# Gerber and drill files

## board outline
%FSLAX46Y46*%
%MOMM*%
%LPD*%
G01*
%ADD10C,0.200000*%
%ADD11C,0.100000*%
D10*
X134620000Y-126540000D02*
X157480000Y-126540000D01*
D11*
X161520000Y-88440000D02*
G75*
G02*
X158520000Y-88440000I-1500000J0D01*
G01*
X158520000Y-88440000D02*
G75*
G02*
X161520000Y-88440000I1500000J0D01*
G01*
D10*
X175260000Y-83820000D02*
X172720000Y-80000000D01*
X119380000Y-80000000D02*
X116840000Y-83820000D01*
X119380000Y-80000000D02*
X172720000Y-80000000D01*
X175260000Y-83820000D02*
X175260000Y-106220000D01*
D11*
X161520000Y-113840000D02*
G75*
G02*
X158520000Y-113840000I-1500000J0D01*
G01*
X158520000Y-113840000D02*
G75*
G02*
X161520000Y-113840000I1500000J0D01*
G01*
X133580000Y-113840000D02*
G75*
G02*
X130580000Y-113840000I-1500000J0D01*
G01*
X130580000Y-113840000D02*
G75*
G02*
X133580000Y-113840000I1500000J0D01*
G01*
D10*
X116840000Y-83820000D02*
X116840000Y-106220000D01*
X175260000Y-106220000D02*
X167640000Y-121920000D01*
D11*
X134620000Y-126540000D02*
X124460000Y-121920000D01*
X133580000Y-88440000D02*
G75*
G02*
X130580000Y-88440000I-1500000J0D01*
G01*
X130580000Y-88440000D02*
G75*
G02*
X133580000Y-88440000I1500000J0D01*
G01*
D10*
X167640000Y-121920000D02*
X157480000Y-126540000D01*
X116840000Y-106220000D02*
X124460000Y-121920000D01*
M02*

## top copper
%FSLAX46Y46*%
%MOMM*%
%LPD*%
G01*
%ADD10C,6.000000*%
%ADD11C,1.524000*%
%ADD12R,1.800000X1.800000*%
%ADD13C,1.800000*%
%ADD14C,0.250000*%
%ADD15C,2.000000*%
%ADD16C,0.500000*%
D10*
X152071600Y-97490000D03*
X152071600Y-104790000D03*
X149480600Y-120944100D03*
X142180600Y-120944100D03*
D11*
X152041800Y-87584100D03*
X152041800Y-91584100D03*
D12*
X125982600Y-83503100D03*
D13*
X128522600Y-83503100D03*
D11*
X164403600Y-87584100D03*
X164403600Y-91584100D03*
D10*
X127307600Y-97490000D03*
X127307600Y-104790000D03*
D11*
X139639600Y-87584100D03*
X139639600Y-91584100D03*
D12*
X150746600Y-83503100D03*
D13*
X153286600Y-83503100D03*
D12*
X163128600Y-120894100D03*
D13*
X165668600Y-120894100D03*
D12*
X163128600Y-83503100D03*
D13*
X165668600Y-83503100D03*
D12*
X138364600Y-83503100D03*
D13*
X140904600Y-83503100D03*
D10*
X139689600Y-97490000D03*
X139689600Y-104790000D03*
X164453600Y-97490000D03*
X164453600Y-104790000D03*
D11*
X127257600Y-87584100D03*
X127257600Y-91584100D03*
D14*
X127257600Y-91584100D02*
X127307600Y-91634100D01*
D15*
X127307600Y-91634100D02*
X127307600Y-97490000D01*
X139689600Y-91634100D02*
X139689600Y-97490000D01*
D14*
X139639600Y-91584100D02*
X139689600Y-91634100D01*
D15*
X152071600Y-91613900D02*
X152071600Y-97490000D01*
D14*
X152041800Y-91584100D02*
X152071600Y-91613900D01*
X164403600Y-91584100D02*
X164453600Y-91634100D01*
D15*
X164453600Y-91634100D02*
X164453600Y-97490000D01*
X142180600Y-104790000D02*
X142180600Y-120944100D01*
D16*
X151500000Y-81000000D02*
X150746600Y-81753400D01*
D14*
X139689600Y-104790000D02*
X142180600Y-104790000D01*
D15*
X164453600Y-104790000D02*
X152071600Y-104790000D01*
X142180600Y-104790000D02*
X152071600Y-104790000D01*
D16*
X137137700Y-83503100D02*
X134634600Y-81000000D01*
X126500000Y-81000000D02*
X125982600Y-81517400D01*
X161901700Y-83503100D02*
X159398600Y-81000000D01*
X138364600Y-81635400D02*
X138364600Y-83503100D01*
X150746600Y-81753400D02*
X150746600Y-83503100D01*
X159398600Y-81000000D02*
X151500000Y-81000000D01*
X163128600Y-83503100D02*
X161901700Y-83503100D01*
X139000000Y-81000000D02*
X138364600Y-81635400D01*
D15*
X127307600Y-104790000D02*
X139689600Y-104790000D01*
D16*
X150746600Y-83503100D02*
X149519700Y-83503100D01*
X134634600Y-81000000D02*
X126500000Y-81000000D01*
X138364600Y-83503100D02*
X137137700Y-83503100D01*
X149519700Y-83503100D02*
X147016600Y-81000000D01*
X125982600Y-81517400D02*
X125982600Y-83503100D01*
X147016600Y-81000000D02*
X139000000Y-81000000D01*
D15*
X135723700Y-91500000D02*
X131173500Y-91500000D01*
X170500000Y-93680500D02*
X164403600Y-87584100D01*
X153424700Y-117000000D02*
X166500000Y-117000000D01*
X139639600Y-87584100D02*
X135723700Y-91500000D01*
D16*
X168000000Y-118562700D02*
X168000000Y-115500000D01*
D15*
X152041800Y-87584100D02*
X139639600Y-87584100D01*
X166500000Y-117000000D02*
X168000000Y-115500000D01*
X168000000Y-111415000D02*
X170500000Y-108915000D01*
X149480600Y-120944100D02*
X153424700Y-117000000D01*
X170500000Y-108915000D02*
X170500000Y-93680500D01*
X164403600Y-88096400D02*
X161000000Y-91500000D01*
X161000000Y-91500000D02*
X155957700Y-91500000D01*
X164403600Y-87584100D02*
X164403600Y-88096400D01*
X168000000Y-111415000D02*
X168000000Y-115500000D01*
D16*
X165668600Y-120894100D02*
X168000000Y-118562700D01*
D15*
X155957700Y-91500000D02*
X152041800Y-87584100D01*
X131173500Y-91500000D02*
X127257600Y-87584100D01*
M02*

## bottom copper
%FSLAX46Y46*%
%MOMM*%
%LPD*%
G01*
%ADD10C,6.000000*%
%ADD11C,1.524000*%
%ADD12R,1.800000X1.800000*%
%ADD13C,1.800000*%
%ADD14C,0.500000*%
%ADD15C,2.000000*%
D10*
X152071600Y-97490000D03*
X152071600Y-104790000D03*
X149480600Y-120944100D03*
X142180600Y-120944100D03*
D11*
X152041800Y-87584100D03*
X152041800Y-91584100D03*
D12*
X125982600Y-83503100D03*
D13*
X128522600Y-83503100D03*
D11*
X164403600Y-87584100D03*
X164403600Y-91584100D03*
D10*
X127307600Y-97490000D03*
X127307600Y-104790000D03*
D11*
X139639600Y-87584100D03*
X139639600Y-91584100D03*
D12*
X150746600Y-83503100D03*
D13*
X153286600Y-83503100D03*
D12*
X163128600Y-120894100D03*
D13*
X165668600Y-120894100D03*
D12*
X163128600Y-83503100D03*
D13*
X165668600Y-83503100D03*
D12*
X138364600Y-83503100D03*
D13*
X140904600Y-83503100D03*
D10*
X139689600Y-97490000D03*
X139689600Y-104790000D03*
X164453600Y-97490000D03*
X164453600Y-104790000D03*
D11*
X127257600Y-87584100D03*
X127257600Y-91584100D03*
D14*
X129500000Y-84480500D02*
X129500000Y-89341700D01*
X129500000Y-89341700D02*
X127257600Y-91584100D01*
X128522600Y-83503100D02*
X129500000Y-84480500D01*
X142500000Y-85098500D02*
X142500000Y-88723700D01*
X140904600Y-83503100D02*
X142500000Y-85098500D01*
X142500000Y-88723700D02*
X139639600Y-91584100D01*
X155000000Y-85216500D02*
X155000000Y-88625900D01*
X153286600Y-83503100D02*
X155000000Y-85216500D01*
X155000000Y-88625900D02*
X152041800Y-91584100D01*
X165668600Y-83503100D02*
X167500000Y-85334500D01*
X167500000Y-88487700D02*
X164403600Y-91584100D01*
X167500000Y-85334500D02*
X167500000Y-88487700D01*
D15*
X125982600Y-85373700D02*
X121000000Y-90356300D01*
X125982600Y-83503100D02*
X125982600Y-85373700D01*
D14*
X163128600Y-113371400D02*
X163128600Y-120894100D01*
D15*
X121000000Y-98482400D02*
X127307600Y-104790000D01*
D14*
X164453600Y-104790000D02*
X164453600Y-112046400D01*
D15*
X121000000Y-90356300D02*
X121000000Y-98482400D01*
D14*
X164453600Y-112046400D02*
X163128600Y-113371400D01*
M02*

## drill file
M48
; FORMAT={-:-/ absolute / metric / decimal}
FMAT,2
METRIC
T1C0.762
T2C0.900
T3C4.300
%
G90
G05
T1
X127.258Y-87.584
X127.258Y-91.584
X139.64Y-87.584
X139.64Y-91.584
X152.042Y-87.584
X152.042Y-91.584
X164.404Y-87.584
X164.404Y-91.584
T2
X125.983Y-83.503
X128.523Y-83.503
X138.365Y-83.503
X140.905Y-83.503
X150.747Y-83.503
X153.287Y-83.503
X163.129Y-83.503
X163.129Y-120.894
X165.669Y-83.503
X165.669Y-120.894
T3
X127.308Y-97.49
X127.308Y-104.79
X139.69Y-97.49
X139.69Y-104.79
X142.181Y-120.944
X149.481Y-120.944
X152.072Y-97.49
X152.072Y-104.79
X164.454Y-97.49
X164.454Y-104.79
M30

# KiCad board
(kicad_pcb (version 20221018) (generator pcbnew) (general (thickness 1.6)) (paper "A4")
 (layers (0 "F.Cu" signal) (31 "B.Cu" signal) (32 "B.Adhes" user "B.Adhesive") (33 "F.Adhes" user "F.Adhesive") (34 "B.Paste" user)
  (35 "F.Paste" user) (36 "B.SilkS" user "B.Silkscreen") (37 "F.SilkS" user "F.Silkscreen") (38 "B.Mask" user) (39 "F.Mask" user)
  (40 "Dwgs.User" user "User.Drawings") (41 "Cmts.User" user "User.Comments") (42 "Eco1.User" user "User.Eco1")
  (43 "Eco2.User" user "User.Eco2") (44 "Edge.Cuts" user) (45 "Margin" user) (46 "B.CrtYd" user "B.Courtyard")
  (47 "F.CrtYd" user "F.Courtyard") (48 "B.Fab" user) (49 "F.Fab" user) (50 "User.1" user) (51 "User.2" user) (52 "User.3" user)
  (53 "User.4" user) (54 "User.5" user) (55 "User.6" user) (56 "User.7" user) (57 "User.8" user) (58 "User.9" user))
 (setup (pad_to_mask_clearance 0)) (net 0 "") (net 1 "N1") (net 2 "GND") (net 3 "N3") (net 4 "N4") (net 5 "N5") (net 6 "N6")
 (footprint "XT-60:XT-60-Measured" (layer "F.Cu") (at 152.0216 101.14 -90)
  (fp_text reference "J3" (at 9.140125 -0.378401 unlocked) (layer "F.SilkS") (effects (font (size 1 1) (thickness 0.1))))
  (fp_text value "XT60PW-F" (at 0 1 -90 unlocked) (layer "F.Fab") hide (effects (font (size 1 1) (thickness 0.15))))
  (pad "1" thru_hole circle (at -3.65 -0.05 270) (size 6 6) (drill 4.3) (layers "*.Cu" "*.Mask") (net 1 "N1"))
  (pad "2" thru_hole circle (at 3.65 -0.05 270) (size 6 6) (drill 4.3) (layers "*.Cu" "*.Mask") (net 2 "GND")))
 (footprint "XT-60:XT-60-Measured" (layer "F.Cu") (at 145.8306 120.8941 180)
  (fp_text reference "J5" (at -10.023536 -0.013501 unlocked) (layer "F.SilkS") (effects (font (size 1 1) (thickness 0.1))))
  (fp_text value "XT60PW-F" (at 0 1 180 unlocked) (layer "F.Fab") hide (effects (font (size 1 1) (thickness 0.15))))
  (pad "1" thru_hole circle (at -3.65 -0.05 180) (size 6 6) (drill 4.3) (layers "*.Cu" "*.Mask") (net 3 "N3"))
  (pad "2" thru_hole circle (at 3.65 -0.05 180) (size 6 6) (drill 4.3) (layers "*.Cu" "*.Mask") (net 2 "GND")))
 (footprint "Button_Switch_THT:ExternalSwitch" (layer "F.Cu") (at 152.0418 89.5841)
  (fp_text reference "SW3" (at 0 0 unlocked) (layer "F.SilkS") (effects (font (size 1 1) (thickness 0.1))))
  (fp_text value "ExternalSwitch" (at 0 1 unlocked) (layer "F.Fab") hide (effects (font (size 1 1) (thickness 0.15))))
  (pad "1" thru_hole circle (at 0 -2) (size 1.524 1.524) (drill 0.762) (layers "*.Cu" "*.Mask") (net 3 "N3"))
  (pad "2" thru_hole circle (at 0 2) (size 1.524 1.524) (drill 0.762) (layers "*.Cu" "*.Mask") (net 1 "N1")))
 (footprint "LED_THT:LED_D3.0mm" (layer "F.Cu") (at 125.9826 83.5031)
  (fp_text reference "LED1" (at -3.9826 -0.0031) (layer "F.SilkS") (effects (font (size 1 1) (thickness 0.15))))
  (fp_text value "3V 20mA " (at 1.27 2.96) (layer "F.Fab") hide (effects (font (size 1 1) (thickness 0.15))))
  (pad "1" thru_hole rect (at 0 0) (size 1.8 1.8) (drill 0.9) (layers "*.Cu" "*.Mask") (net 2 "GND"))
  (pad "2" thru_hole circle (at 2.54 0) (size 1.8 1.8) (drill 0.9) (layers "*.Cu" "*.Mask") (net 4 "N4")))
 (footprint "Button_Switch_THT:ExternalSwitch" (layer "F.Cu") (at 164.4036 89.5841)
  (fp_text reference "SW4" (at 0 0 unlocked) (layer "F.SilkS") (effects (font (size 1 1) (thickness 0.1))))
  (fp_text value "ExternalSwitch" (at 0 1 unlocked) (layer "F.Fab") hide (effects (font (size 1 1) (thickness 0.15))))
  (pad "1" thru_hole circle (at 0 -2) (size 1.524 1.524) (drill 0.762) (layers "*.Cu" "*.Mask") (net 3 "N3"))
  (pad "2" thru_hole circle (at 0 2) (size 1.524 1.524) (drill 0.762) (layers "*.Cu" "*.Mask") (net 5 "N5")))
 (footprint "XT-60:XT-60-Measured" (layer "F.Cu") (at 127.2576 101.14 -90)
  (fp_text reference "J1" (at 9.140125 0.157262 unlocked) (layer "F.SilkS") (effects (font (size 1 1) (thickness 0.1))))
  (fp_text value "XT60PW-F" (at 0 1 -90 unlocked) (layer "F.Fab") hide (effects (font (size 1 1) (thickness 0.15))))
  (pad "1" thru_hole circle (at -3.65 -0.05 270) (size 6 6) (drill 4.3) (layers "*.Cu" "*.Mask") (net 4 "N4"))
  (pad "2" thru_hole circle (at 3.65 -0.05 270) (size 6 6) (drill 4.3) (layers "*.Cu" "*.Mask") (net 2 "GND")))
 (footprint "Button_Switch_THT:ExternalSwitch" (layer "F.Cu") (at 139.6396 89.5841)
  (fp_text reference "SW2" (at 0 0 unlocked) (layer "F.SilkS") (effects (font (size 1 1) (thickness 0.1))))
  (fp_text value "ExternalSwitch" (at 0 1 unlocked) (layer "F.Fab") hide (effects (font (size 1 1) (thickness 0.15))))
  (pad "1" thru_hole circle (at 0 -2) (size 1.524 1.524) (drill 0.762) (layers "*.Cu" "*.Mask") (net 3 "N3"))
  (pad "2" thru_hole circle (at 0 2) (size 1.524 1.524) (drill 0.762) (layers "*.Cu" "*.Mask") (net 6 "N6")))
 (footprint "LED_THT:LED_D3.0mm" (layer "F.Cu") (at 150.7466 83.5031)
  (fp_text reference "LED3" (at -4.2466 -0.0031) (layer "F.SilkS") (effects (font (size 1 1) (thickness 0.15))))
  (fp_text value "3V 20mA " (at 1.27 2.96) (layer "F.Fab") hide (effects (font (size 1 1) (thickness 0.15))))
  (pad "1" thru_hole rect (at 0 0) (size 1.8 1.8) (drill 0.9) (layers "*.Cu" "*.Mask") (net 2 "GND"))
  (pad "2" thru_hole circle (at 2.54 0) (size 1.8 1.8) (drill 0.9) (layers "*.Cu" "*.Mask") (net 1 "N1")))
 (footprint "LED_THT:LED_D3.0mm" (layer "F.Cu") (at 163.1286 120.8941)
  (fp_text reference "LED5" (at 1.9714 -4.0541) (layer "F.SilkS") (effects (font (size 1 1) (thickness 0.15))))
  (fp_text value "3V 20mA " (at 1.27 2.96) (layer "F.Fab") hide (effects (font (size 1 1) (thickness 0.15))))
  (pad "1" thru_hole rect (at 0 0) (size 1.8 1.8) (drill 0.9) (layers "*.Cu" "*.Mask") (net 2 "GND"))
  (pad "2" thru_hole circle (at 2.54 0) (size 1.8 1.8) (drill 0.9) (layers "*.Cu" "*.Mask") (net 3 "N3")))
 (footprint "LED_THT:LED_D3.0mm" (layer "F.Cu") (at 163.1286 83.5031)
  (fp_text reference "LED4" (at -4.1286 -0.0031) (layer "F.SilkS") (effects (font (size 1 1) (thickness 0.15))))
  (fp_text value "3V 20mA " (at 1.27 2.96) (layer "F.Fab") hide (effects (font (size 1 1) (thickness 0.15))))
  (pad "1" thru_hole rect (at 0 0) (size 1.8 1.8) (drill 0.9) (layers "*.Cu" "*.Mask") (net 2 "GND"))
  (pad "2" thru_hole circle (at 2.54 0) (size 1.8 1.8) (drill 0.9) (layers "*.Cu" "*.Mask") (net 5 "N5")))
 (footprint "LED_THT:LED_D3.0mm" (layer "F.Cu") (at 138.3646 83.5031)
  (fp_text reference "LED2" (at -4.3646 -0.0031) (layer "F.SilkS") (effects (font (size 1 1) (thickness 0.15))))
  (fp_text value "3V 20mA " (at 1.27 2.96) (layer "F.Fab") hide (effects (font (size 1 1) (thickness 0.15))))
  (pad "1" thru_hole rect (at 0 0) (size 1.8 1.8) (drill 0.9) (layers "*.Cu" "*.Mask") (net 2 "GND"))
  (pad "2" thru_hole circle (at 2.54 0) (size 1.8 1.8) (drill 0.9) (layers "*.Cu" "*.Mask") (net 6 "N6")))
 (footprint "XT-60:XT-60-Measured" (layer "F.Cu") (at 139.6396 101.14 -90)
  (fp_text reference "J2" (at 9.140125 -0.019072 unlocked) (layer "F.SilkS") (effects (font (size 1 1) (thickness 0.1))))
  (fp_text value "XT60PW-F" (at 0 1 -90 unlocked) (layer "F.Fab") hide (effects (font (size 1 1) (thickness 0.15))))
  (pad "1" thru_hole circle (at -3.65 -0.05 270) (size 6 6) (drill 4.3) (layers "*.Cu" "*.Mask") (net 6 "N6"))
  (pad "2" thru_hole circle (at 3.65 -0.05 270) (size 6 6) (drill 4.3) (layers "*.Cu" "*.Mask") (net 2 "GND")))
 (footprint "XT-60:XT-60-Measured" (layer "F.Cu") (at 164.4036 101.14 -90)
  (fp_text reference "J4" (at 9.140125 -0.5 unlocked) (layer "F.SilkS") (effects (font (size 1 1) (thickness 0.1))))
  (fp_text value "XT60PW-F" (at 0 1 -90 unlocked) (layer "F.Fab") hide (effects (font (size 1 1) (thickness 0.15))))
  (pad "1" thru_hole circle (at -3.65 -0.05 270) (size 6 6) (drill 4.3) (layers "*.Cu" "*.Mask") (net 5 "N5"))
  (pad "2" thru_hole circle (at 3.65 -0.05 270) (size 6 6) (drill 4.3) (layers "*.Cu" "*.Mask") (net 2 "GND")))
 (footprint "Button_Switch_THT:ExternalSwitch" (layer "F.Cu") (at 127.2576 89.5841)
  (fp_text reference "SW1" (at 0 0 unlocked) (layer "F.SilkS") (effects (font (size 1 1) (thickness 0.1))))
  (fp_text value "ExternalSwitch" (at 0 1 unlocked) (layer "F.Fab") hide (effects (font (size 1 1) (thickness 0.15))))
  (pad "1" thru_hole circle (at 0 -2) (size 1.524 1.524) (drill 0.762) (layers "*.Cu" "*.Mask") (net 3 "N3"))
  (pad "2" thru_hole circle (at 0 2) (size 1.524 1.524) (drill 0.762) (layers "*.Cu" "*.Mask") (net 4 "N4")))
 (gr_line (start 134.62 126.54) (end 157.48 126.54) (stroke (width 0.2) (type default)) (layer "Edge.Cuts"))
 (gr_circle (center 160.02 88.44) (end 161.52 88.44) (stroke (width 0.1) (type default)) (fill none) (layer "Edge.Cuts"))
 (gr_line (start 175.26 83.82) (end 172.72 80) (stroke (width 0.2) (type default)) (layer "Edge.Cuts"))
 (gr_line (start 119.38 80) (end 116.84 83.82) (stroke (width 0.2) (type default)) (layer "Edge.Cuts"))
 (gr_line (start 119.38 80) (end 172.72 80) (stroke (width 0.2) (type default)) (layer "Edge.Cuts"))
 (gr_line (start 175.26 83.82) (end 175.26 106.22) (stroke (width 0.2) (type default)) (layer "Edge.Cuts"))
 (gr_circle (center 160.02 113.84) (end 161.52 113.84) (stroke (width 0.1) (type default)) (fill none) (layer "Edge.Cuts"))
 (gr_circle (center 132.08 113.84) (end 133.58 113.84) (stroke (width 0.1) (type default)) (fill none) (layer "Edge.Cuts"))
 (gr_line (start 116.84 83.82) (end 116.84 106.22) (stroke (width 0.2) (type default)) (layer "Edge.Cuts"))
 (gr_line (start 175.26 106.22) (end 167.64 121.92) (stroke (width 0.2) (type default)) (layer "Edge.Cuts"))
 (gr_line (start 134.62 126.54) (end 124.46 121.92) (stroke (width 0.1) (type default)) (layer "Edge.Cuts"))
 (gr_circle (center 132.08 88.44) (end 133.58 88.44) (stroke (width 0.1) (type default)) (fill none) (layer "Edge.Cuts"))
 (gr_line (start 167.64 121.92) (end 157.48 126.54) (stroke (width 0.2) (type default)) (layer "Edge.Cuts"))
 (gr_line (start 116.84 106.22) (end 124.46 121.92) (stroke (width 0.2) (type default)) (layer "Edge.Cuts"))
 (segment (start 127.2576 91.5841) (end 127.3076 91.6341) (width 0.25) (layer "F.Cu") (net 4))
 (segment (start 127.3076 91.6341) (end 127.3076 97.49) (width 2) (layer "F.Cu") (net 4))
 (segment (start 129.5 84.4805) (end 129.5 89.3417) (width 0.5) (layer "B.Cu") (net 4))
 (segment (start 129.5 89.3417) (end 127.2576 91.5841) (width 0.5) (layer "B.Cu") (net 4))
 (segment (start 128.5226 83.5031) (end 129.5 84.4805) (width 0.5) (layer "B.Cu") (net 4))
 (segment (start 139.6896 91.6341) (end 139.6896 97.49) (width 2) (layer "F.Cu") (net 6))
 (segment (start 139.6396 91.5841) (end 139.6896 91.6341) (width 0.25) (layer "F.Cu") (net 6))
 (segment (start 142.5 85.0985) (end 142.5 88.7237) (width 0.5) (layer "B.Cu") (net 6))
 (segment (start 140.9046 83.5031) (end 142.5 85.0985) (width 0.5) (layer "B.Cu") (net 6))
 (segment (start 142.5 88.7237) (end 139.6396 91.5841) (width 0.5) (layer "B.Cu") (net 6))
 (segment (start 152.0716 91.6139) (end 152.0716 97.49) (width 2) (layer "F.Cu") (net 1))
 (segment (start 152.0418 91.5841) (end 152.0716 91.6139) (width 0.25) (layer "F.Cu") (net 1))
 (segment (start 155 85.2165) (end 155 88.6259) (width 0.5) (layer "B.Cu") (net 1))
 (segment (start 153.2866 83.5031) (end 155 85.2165) (width 0.5) (layer "B.Cu") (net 1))
 (segment (start 155 88.6259) (end 152.0418 91.5841) (width 0.5) (layer "B.Cu") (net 1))
 (segment (start 164.4036 91.5841) (end 164.4536 91.6341) (width 0.25) (layer "F.Cu") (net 5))
 (segment (start 164.4536 91.6341) (end 164.4536 97.49) (width 2) (layer "F.Cu") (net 5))
 (segment (start 165.6686 83.5031) (end 167.5 85.3345) (width 0.5) (layer "B.Cu") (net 5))
 (segment (start 167.5 88.4877) (end 164.4036 91.5841) (width 0.5) (layer "B.Cu") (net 5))
 (segment (start 167.5 85.3345) (end 167.5 88.4877) (width 0.5) (layer "B.Cu") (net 5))
 (segment (start 142.1806 104.79) (end 142.1806 120.9441) (width 2) (layer "F.Cu") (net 2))
 (segment (start 151.5 81) (end 150.7466 81.7534) (width 0.5) (layer "F.Cu") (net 2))
 (segment (start 139.6896 104.79) (end 142.1806 104.79) (width 0.25) (layer "F.Cu") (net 2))
 (segment (start 164.4536 104.79) (end 152.0716 104.79) (width 2) (layer "F.Cu") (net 2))
 (segment (start 142.1806 104.79) (end 152.0716 104.79) (width 2) (layer "F.Cu") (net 2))
 (segment (start 137.1377 83.5031) (end 134.6346 81) (width 0.5) (layer "F.Cu") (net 2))
 (segment (start 126.5 81) (end 125.9826 81.5174) (width 0.5) (layer "F.Cu") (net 2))
 (segment (start 161.9017 83.5031) (end 159.3986 81) (width 0.5) (layer "F.Cu") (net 2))
 (segment (start 138.3646 81.6354) (end 138.3646 83.5031) (width 0.5) (layer "F.Cu") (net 2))
 (segment (start 150.7466 81.7534) (end 150.7466 83.5031) (width 0.5) (layer "F.Cu") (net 2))
 (segment (start 159.3986 81) (end 151.5 81) (width 0.5) (layer "F.Cu") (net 2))
 (segment (start 163.1286 83.5031) (end 161.9017 83.5031) (width 0.5) (layer "F.Cu") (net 2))
 (segment (start 139 81) (end 138.3646 81.6354) (width 0.5) (layer "F.Cu") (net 2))
 (segment (start 127.3076 104.79) (end 139.6896 104.79) (width 2) (layer "F.Cu") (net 2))
 (segment (start 150.7466 83.5031) (end 149.5197 83.5031) (width 0.5) (layer "F.Cu") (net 2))
 (segment (start 134.6346 81) (end 126.5 81) (width 0.5) (layer "F.Cu") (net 2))
 (segment (start 138.3646 83.5031) (end 137.1377 83.5031) (width 0.5) (layer "F.Cu") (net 2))
 (segment (start 149.5197 83.5031) (end 147.0166 81) (width 0.5) (layer "F.Cu") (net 2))
 (segment (start 125.9826 81.5174) (end 125.9826 83.5031) (width 0.5) (layer "F.Cu") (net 2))
 (segment (start 147.0166 81) (end 139 81) (width 0.5) (layer "F.Cu") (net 2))
 (segment (start 125.9826 85.3737) (end 121 90.3563) (width 2) (layer "B.Cu") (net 2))
 (segment (start 125.9826 83.5031) (end 125.9826 85.3737) (width 2) (layer "B.Cu") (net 2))
 (segment (start 163.1286 113.3714) (end 163.1286 120.8941) (width 0.5) (layer "B.Cu") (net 2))
 (segment (start 121 98.4824) (end 127.3076 104.79) (width 2) (layer "B.Cu") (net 2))
 (segment (start 164.4536 104.79) (end 164.4536 112.0464) (width 0.5) (layer "B.Cu") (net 2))
 (segment (start 121 90.3563) (end 121 98.4824) (width 2) (layer "B.Cu") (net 2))
 (segment (start 164.4536 112.0464) (end 163.1286 113.3714) (width 0.5) (layer "B.Cu") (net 2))
 (segment (start 135.7237 91.5) (end 131.1735 91.5) (width 2) (layer "F.Cu") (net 3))
 (segment (start 170.5 93.6805) (end 164.4036 87.5841) (width 2) (layer "F.Cu") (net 3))
 (segment (start 153.4247 117) (end 166.5 117) (width 2) (layer "F.Cu") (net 3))
 (segment (start 139.6396 87.5841) (end 135.7237 91.5) (width 2) (layer "F.Cu") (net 3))
 (segment (start 168 118.5627) (end 168 115.5) (width 0.5) (layer "F.Cu") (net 3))
 (segment (start 152.0418 87.5841) (end 139.6396 87.5841) (width 2) (layer "F.Cu") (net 3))
 (segment (start 166.5 117) (end 168 115.5) (width 2) (layer "F.Cu") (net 3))
 (segment (start 168 111.415) (end 170.5 108.915) (width 2) (layer "F.Cu") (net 3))
 (segment (start 149.4806 120.9441) (end 153.4247 117) (width 2) (layer "F.Cu") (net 3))
 (segment (start 170.5 108.915) (end 170.5 93.6805) (width 2) (layer "F.Cu") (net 3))
 (segment (start 164.4036 88.0964) (end 161 91.5) (width 2) (layer "F.Cu") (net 3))
 (segment (start 161 91.5) (end 155.9577 91.5) (width 2) (layer "F.Cu") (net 3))
 (segment (start 164.4036 87.5841) (end 164.4036 88.0964) (width 2) (layer "F.Cu") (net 3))
 (segment (start 168 111.415) (end 168 115.5) (width 2) (layer "F.Cu") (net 3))
 (segment (start 165.6686 120.8941) (end 168 118.5627) (width 0.5) (layer "F.Cu") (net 3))
 (segment (start 155.9577 91.5) (end 152.0418 87.5841) (width 2) (layer "F.Cu") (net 3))
 (segment (start 131.1735 91.5) (end 127.2576 87.5841) (width 2) (layer "F.Cu") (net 3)))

